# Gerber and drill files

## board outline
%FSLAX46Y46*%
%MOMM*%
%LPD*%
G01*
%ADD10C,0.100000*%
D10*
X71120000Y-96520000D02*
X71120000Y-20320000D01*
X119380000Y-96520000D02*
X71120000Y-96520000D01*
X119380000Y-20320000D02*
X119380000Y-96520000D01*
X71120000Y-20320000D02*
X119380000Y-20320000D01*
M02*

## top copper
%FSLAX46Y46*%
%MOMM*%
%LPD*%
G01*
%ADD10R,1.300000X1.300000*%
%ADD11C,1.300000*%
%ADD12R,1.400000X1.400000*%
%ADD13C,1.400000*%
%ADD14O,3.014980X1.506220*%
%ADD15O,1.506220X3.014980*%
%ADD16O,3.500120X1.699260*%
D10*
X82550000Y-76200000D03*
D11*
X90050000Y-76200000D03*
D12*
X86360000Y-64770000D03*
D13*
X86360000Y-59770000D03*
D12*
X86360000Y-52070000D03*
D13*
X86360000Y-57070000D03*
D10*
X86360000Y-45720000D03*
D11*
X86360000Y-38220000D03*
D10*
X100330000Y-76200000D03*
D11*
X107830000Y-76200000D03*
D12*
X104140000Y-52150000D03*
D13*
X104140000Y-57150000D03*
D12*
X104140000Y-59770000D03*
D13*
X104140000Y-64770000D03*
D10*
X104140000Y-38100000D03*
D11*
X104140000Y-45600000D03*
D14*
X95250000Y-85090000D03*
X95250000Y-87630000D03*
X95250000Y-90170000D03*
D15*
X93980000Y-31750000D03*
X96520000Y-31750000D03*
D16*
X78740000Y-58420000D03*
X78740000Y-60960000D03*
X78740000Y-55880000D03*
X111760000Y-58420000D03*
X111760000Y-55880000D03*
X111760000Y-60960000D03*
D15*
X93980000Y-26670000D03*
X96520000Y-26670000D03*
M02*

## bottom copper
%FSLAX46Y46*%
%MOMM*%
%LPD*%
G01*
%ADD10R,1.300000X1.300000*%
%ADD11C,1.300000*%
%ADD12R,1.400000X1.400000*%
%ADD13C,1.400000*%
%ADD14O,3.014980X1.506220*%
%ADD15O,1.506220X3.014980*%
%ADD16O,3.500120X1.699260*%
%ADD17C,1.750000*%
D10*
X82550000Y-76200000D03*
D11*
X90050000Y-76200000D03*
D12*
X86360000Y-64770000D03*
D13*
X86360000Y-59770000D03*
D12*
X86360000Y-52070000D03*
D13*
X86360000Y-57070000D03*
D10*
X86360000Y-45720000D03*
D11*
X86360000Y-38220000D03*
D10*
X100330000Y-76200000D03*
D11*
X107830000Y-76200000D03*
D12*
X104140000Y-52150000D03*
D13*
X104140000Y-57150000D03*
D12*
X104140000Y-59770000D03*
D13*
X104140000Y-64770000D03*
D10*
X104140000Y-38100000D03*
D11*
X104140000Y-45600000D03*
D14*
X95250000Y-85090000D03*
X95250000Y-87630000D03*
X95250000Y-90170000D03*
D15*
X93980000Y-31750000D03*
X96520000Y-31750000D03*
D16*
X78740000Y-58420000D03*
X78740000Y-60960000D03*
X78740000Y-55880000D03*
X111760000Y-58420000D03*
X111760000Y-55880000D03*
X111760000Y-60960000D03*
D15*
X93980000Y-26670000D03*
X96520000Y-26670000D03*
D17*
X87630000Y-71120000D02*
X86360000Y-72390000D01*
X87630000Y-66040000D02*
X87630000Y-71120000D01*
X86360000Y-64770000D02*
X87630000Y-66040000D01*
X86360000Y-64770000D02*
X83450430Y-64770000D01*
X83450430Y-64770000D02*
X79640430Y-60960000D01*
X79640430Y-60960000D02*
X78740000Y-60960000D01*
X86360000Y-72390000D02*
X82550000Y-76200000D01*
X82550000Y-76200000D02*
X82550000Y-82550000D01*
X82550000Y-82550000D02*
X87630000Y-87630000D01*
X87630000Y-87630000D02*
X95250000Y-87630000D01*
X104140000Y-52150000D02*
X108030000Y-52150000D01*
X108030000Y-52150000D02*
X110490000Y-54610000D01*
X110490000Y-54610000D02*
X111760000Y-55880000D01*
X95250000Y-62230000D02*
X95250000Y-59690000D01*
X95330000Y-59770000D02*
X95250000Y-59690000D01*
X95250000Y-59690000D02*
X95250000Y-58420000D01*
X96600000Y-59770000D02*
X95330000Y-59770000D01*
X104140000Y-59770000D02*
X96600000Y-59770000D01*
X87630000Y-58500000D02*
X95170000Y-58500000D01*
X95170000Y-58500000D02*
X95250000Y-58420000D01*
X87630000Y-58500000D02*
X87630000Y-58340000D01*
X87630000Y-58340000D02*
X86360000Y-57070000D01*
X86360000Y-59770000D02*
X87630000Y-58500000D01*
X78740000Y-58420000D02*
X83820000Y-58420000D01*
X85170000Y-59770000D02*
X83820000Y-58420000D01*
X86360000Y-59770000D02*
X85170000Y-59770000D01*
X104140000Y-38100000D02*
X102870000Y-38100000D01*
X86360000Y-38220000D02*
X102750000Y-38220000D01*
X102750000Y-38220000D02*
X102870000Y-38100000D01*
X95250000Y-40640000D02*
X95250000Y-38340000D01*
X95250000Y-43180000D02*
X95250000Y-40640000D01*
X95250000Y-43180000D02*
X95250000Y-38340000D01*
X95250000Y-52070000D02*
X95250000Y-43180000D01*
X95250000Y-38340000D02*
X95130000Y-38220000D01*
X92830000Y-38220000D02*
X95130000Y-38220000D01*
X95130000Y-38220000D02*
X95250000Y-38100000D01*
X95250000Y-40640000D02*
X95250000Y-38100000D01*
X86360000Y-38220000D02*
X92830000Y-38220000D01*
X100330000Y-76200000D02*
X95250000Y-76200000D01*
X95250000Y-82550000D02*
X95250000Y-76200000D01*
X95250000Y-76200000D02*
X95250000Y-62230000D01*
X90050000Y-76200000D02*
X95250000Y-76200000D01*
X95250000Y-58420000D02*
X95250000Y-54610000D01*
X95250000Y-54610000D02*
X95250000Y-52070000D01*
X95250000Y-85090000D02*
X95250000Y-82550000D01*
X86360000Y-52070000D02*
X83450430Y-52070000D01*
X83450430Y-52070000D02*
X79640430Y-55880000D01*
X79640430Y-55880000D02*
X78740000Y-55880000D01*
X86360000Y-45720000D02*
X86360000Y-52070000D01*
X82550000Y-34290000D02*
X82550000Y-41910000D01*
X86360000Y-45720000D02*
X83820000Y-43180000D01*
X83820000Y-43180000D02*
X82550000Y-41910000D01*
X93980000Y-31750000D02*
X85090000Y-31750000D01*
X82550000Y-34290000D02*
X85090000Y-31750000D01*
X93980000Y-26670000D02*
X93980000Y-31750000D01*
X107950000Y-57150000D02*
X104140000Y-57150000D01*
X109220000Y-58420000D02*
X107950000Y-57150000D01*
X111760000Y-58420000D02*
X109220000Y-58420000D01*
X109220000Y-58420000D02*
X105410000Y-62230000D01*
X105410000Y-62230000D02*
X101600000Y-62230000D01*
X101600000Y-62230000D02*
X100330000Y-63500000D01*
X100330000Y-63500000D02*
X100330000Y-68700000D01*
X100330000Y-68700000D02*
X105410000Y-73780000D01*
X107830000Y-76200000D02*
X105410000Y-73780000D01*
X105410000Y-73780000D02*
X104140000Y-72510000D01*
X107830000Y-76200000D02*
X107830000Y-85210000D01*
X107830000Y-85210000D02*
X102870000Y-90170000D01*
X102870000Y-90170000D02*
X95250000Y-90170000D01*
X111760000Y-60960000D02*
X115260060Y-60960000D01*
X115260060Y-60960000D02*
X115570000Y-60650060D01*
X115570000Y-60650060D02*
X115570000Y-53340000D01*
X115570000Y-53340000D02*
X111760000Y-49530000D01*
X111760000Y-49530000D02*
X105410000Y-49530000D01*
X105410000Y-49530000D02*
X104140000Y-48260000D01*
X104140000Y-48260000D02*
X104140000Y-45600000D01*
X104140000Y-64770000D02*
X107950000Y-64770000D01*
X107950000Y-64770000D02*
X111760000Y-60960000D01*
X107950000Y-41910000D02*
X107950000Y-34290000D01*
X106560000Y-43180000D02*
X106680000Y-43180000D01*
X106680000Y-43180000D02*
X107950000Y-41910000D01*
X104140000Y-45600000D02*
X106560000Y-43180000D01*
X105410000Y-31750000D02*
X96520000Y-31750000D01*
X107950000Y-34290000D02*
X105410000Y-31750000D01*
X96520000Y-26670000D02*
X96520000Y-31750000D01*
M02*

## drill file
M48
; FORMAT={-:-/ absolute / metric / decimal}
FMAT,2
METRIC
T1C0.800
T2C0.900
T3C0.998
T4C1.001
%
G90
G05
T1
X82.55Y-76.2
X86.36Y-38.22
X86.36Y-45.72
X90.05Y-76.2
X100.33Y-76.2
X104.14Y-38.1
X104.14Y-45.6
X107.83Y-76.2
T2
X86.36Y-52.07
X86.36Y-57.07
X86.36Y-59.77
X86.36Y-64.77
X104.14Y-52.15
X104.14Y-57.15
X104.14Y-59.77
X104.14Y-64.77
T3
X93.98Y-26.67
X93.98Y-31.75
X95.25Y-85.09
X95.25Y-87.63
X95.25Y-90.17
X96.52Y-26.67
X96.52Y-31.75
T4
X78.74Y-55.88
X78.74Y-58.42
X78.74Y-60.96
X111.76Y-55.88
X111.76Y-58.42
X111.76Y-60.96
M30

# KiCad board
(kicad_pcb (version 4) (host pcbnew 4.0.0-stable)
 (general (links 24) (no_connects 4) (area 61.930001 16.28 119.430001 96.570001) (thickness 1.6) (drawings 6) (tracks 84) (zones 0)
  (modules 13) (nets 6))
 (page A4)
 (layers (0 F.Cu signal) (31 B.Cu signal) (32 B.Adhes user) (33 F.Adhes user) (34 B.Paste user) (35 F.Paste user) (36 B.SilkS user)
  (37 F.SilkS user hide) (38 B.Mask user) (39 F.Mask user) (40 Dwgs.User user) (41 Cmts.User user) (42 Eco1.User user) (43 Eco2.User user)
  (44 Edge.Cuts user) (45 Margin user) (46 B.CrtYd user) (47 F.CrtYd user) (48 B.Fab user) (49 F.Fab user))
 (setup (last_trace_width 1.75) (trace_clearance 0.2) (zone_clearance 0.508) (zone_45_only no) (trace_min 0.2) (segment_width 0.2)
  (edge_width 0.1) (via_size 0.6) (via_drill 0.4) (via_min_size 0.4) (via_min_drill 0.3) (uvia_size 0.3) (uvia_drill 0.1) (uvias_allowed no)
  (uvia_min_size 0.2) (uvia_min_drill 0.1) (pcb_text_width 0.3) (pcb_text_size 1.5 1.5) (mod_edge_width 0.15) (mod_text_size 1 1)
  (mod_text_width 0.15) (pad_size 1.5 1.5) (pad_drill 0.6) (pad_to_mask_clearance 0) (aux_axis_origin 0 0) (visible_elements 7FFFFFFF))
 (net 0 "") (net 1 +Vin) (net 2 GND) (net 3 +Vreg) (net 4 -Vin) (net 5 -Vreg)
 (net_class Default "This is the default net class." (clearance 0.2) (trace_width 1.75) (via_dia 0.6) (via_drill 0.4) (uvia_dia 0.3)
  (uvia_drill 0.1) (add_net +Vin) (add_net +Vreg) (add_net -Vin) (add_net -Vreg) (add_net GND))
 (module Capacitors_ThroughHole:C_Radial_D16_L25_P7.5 (layer F.Cu) (at 82.55 76.2)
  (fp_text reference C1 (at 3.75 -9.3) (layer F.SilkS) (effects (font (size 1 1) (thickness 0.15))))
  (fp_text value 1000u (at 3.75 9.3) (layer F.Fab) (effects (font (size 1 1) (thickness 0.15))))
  (pad 1 thru_hole rect (at 0 0) (size 1.3 1.3) (drill 0.8) (layers *.Cu *.Mask F.SilkS) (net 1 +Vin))
  (pad 2 thru_hole circle (at 7.5 0) (size 1.3 1.3) (drill 0.8) (layers *.Cu *.Mask F.SilkS) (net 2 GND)))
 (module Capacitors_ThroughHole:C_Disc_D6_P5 (layer F.Cu) (at 86.36 64.77 90)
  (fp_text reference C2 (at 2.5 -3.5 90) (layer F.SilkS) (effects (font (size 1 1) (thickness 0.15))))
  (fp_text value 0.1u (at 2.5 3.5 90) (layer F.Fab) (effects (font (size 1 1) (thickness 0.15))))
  (pad 1 thru_hole rect (at 0 0 90) (size 1.4 1.4) (drill 0.9) (layers *.Cu *.Mask F.SilkS) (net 1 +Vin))
  (pad 2 thru_hole circle (at 5 0 90) (size 1.4 1.4) (drill 0.9) (layers *.Cu *.Mask F.SilkS) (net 2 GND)))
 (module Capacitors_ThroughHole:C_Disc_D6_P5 (layer F.Cu) (at 86.36 52.07 270)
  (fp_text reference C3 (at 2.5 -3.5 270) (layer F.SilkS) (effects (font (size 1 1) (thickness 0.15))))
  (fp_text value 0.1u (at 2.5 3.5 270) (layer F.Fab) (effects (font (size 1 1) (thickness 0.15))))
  (pad 1 thru_hole rect (at 0 0 270) (size 1.4 1.4) (drill 0.9) (layers *.Cu *.Mask F.SilkS) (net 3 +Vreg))
  (pad 2 thru_hole circle (at 5 0 270) (size 1.4 1.4) (drill 0.9) (layers *.Cu *.Mask F.SilkS) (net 2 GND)))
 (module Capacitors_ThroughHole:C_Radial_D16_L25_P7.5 (layer F.Cu) (at 86.36 45.72 90)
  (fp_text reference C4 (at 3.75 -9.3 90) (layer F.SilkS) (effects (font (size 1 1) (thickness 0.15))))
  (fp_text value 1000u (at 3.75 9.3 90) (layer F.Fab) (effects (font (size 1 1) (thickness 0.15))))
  (pad 1 thru_hole rect (at 0 0 90) (size 1.3 1.3) (drill 0.8) (layers *.Cu *.Mask F.SilkS) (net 3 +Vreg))
  (pad 2 thru_hole circle (at 7.5 0 90) (size 1.3 1.3) (drill 0.8) (layers *.Cu *.Mask F.SilkS) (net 2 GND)))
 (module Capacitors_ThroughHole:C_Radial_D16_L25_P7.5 (layer F.Cu) (at 100.33 76.2)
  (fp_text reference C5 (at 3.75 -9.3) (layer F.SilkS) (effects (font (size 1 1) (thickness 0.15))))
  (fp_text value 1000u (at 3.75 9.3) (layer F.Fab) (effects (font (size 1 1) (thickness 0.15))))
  (pad 1 thru_hole rect (at 0 0) (size 1.3 1.3) (drill 0.8) (layers *.Cu *.Mask F.SilkS) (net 2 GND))
  (pad 2 thru_hole circle (at 7.5 0) (size 1.3 1.3) (drill 0.8) (layers *.Cu *.Mask F.SilkS) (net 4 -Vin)))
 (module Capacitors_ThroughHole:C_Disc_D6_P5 (layer F.Cu) (at 104.14 52.15 270)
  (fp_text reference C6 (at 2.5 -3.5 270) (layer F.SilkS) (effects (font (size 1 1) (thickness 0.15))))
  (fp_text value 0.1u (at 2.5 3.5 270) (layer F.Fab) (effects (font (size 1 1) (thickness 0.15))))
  (pad 1 thru_hole rect (at 0 0 270) (size 1.4 1.4) (drill 0.9) (layers *.Cu *.Mask F.SilkS) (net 2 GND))
  (pad 2 thru_hole circle (at 5 0 270) (size 1.4 1.4) (drill 0.9) (layers *.Cu *.Mask F.SilkS) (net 4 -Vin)))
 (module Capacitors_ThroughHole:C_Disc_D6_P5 (layer F.Cu) (at 104.14 59.77 270)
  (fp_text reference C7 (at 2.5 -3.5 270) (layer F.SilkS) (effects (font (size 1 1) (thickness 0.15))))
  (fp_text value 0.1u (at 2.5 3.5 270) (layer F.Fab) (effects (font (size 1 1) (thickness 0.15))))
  (pad 1 thru_hole rect (at 0 0 270) (size 1.4 1.4) (drill 0.9) (layers *.Cu *.Mask F.SilkS) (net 2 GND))
  (pad 2 thru_hole circle (at 5 0 270) (size 1.4 1.4) (drill 0.9) (layers *.Cu *.Mask F.SilkS) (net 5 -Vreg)))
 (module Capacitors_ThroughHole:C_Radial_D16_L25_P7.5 (layer F.Cu) (at 104.14 38.1 270)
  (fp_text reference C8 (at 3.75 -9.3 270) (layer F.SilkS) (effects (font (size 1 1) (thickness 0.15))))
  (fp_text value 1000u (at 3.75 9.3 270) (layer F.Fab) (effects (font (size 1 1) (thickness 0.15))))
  (pad 1 thru_hole rect (at 0 0 270) (size 1.3 1.3) (drill 0.8) (layers *.Cu *.Mask F.SilkS) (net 2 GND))
  (pad 2 thru_hole circle (at 7.5 0 270) (size 1.3 1.3) (drill 0.8) (layers *.Cu *.Mask F.SilkS) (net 5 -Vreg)))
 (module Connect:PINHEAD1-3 (layer F.Cu) (at 95.25 87.63 270)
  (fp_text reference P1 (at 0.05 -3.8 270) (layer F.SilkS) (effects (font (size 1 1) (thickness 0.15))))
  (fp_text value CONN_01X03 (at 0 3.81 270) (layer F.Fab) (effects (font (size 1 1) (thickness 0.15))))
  (pad 1 thru_hole oval (at -2.54 0 270) (size 1.50622 3.01498) (drill 0.99822) (layers *.Cu *.Mask) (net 2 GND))
  (pad 2 thru_hole oval (at 0 0 270) (size 1.50622 3.01498) (drill 0.99822) (layers *.Cu *.Mask) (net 1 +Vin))
  (pad 3 thru_hole oval (at 2.54 0 270) (size 1.50622 3.01498) (drill 0.99822) (layers *.Cu *.Mask) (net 4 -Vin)))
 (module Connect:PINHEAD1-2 (layer F.Cu) (at 95.25 31.75)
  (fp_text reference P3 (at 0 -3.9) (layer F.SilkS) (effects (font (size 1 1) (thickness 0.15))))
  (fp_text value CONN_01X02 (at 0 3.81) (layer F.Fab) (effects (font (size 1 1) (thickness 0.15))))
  (pad 1 thru_hole oval (at -1.27 0) (size 1.50622 3.01498) (drill 0.99822) (layers *.Cu *.Mask) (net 3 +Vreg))
  (pad 2 thru_hole oval (at 1.27 0) (size 1.50622 3.01498) (drill 0.99822) (layers *.Cu *.Mask) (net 5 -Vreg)))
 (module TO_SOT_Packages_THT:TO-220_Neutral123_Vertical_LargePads (layer F.Cu) (at 78.74 58.42 90)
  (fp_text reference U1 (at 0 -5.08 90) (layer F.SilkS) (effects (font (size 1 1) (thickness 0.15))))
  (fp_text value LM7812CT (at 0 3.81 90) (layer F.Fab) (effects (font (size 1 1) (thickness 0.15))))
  (pad 2 thru_hole oval (at 0 0 180) (size 3.50012 1.69926) (drill 1.00076) (layers *.Cu *.Mask F.SilkS) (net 2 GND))
  (pad 1 thru_hole oval (at -2.54 0 180) (size 3.50012 1.69926) (drill 1.00076) (layers *.Cu *.Mask F.SilkS) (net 1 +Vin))
  (pad 3 thru_hole oval (at 2.54 0 180) (size 3.50012 1.69926) (drill 1.00076) (layers *.Cu *.Mask F.SilkS) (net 3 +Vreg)))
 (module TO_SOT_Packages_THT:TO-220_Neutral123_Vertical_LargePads (layer F.Cu) (at 111.76 58.42 270)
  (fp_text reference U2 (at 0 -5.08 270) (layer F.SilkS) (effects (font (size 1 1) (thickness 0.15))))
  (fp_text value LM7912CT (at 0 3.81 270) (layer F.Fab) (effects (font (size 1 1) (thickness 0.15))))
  (pad 2 thru_hole oval (at 0 0) (size 3.50012 1.69926) (drill 1.00076) (layers *.Cu *.Mask F.SilkS) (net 4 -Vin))
  (pad 1 thru_hole oval (at -2.54 0) (size 3.50012 1.69926) (drill 1.00076) (layers *.Cu *.Mask F.SilkS) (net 2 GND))
  (pad 3 thru_hole oval (at 2.54 0) (size 3.50012 1.69926) (drill 1.00076) (layers *.Cu *.Mask F.SilkS) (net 5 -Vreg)))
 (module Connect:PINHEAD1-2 (layer F.Cu) (at 95.25 26.67)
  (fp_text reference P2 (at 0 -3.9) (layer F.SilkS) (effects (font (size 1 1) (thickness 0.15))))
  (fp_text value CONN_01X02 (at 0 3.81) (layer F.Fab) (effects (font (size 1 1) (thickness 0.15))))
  (pad 1 thru_hole oval (at -1.27 0) (size 1.50622 3.01498) (drill 0.99822) (layers *.Cu *.Mask) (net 3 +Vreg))
  (pad 2 thru_hole oval (at 1.27 0) (size 1.50622 3.01498) (drill 0.99822) (layers *.Cu *.Mask) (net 5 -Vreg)))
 (gr_line (start 71.12 96.52) (end 71.12 20.32) (angle 90) (layer Edge.Cuts) (width 0.1))
 (gr_line (start 119.38 96.52) (end 71.12 96.52) (angle 90) (layer Edge.Cuts) (width 0.1))
 (gr_line (start 119.38 20.32) (end 119.38 96.52) (angle 90) (layer Edge.Cuts) (width 0.1))
 (gr_line (start 71.12 20.32) (end 119.38 20.32) (angle 90) (layer Edge.Cuts) (width 0.1))
 (segment (start 87.63 71.12) (end 86.36 72.39) (width 1.75) (layer B.Cu) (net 1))
 (segment (start 87.63 66.04) (end 87.63 71.12) (width 1.75) (layer B.Cu) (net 1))
 (segment (start 86.36 64.77) (end 87.63 66.04) (width 1.75) (layer B.Cu) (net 1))
 (segment (start 86.36 64.77) (end 83.45043 64.77) (width 1.75) (layer B.Cu) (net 1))
 (segment (start 83.45043 64.77) (end 79.64043 60.96) (width 1.75) (layer B.Cu) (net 1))
 (segment (start 79.64043 60.96) (end 78.74 60.96) (width 1.75) (layer B.Cu) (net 1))
 (segment (start 86.36 72.39) (end 82.55 76.2) (width 1.75) (layer B.Cu) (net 1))
 (segment (start 82.55 76.2) (end 82.55 82.55) (width 1.75) (layer B.Cu) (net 1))
 (segment (start 82.55 82.55) (end 87.63 87.63) (width 1.75) (layer B.Cu) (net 1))
 (segment (start 87.63 87.63) (end 95.25 87.63) (width 1.75) (layer B.Cu) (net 1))
 (segment (start 104.14 52.15) (end 108.03 52.15) (width 1.75) (layer B.Cu) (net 2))
 (segment (start 108.03 52.15) (end 110.49 54.61) (width 1.75) (layer B.Cu) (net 2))
 (segment (start 110.49 54.61) (end 111.76 55.88) (width 1.75) (layer B.Cu) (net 2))
 (segment (start 95.25 62.23) (end 95.25 59.69) (width 1.75) (layer B.Cu) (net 2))
 (segment (start 95.33 59.77) (end 95.25 59.69) (width 1.75) (layer B.Cu) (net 2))
 (segment (start 95.25 59.69) (end 95.25 58.42) (width 1.75) (layer B.Cu) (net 2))
 (segment (start 96.6 59.77) (end 95.33 59.77) (width 1.75) (layer B.Cu) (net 2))
 (segment (start 104.14 59.77) (end 96.6 59.77) (width 1.75) (layer B.Cu) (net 2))
 (segment (start 87.63 58.5) (end 95.17 58.5) (width 1.75) (layer B.Cu) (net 2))
 (segment (start 95.17 58.5) (end 95.25 58.42) (width 1.75) (layer B.Cu) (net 2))
 (segment (start 87.63 58.5) (end 87.63 58.34) (width 1.75) (layer B.Cu) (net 2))
 (segment (start 87.63 58.34) (end 86.36 57.07) (width 1.75) (layer B.Cu) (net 2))
 (segment (start 86.36 59.77) (end 87.63 58.5) (width 1.75) (layer B.Cu) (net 2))
 (segment (start 78.74 58.42) (end 83.82 58.42) (width 1.75) (layer B.Cu) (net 2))
 (segment (start 85.17 59.77) (end 83.82 58.42) (width 1.75) (layer B.Cu) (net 2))
 (segment (start 86.36 59.77) (end 85.17 59.77) (width 1.75) (layer B.Cu) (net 2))
 (segment (start 104.14 38.1) (end 102.87 38.1) (width 1.75) (layer B.Cu) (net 2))
 (segment (start 86.36 38.22) (end 102.75 38.22) (width 1.75) (layer B.Cu) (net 2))
 (segment (start 102.75 38.22) (end 102.87 38.1) (width 1.75) (layer B.Cu) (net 2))
 (segment (start 95.25 40.64) (end 95.25 38.34) (width 1.75) (layer B.Cu) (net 2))
 (segment (start 95.25 43.18) (end 95.25 40.64) (width 1.75) (layer B.Cu) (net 2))
 (segment (start 95.25 43.18) (end 95.25 38.34) (width 1.75) (layer B.Cu) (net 2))
 (segment (start 95.25 52.07) (end 95.25 43.18) (width 1.75) (layer B.Cu) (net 2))
 (segment (start 95.25 38.34) (end 95.13 38.22) (width 1.75) (layer B.Cu) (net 2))
 (segment (start 92.83 38.22) (end 95.13 38.22) (width 1.75) (layer B.Cu) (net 2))
 (segment (start 95.13 38.22) (end 95.25 38.1) (width 1.75) (layer B.Cu) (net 2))
 (segment (start 95.25 40.64) (end 95.25 38.1) (width 1.75) (layer B.Cu) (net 2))
 (segment (start 86.36 38.22) (end 92.83 38.22) (width 1.75) (layer B.Cu) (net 2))
 (segment (start 100.33 76.2) (end 95.25 76.2) (width 1.75) (layer B.Cu) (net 2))
 (segment (start 95.25 82.55) (end 95.25 76.2) (width 1.75) (layer B.Cu) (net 2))
 (segment (start 95.25 76.2) (end 95.25 62.23) (width 1.75) (layer B.Cu) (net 2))
 (segment (start 90.05 76.2) (end 95.25 76.2) (width 1.75) (layer B.Cu) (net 2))
 (segment (start 95.25 58.42) (end 95.25 54.61) (width 1.75) (layer B.Cu) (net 2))
 (segment (start 95.25 54.61) (end 95.25 52.07) (width 1.75) (layer B.Cu) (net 2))
 (segment (start 95.25 85.09) (end 95.25 82.55) (width 1.75) (layer B.Cu) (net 2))
 (segment (start 86.36 52.07) (end 83.45043 52.07) (width 1.75) (layer B.Cu) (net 3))
 (segment (start 83.45043 52.07) (end 79.64043 55.88) (width 1.75) (layer B.Cu) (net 3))
 (segment (start 79.64043 55.88) (end 78.74 55.88) (width 1.75) (layer B.Cu) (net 3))
 (segment (start 86.36 45.72) (end 86.36 52.07) (width 1.75) (layer B.Cu) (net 3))
 (segment (start 82.55 34.29) (end 82.55 41.91) (width 1.75) (layer B.Cu) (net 3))
 (segment (start 86.36 45.72) (end 83.82 43.18) (width 1.75) (layer B.Cu) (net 3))
 (segment (start 83.82 43.18) (end 82.55 41.91) (width 1.75) (layer B.Cu) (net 3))
 (segment (start 93.98 31.75) (end 85.09 31.75) (width 1.75) (layer B.Cu) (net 3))
 (segment (start 82.55 34.29) (end 85.09 31.75) (width 1.75) (layer B.Cu) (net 3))
 (segment (start 93.98 26.67) (end 93.98 31.75) (width 1.75) (layer B.Cu) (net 3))
 (segment (start 107.95 57.15) (end 104.14 57.15) (width 1.75) (layer B.Cu) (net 4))
 (segment (start 109.22 58.42) (end 107.95 57.15) (width 1.75) (layer B.Cu) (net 4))
 (segment (start 111.76 58.42) (end 109.22 58.42) (width 1.75) (layer B.Cu) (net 4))
 (segment (start 109.22 58.42) (end 105.41 62.23) (width 1.75) (layer B.Cu) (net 4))
 (segment (start 105.41 62.23) (end 101.6 62.23) (width 1.75) (layer B.Cu) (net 4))
 (segment (start 101.6 62.23) (end 100.33 63.5) (width 1.75) (layer B.Cu) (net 4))
 (segment (start 100.33 63.5) (end 100.33 68.7) (width 1.75) (layer B.Cu) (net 4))
 (segment (start 100.33 68.7) (end 105.41 73.78) (width 1.75) (layer B.Cu) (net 4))
 (segment (start 107.83 76.2) (end 105.41 73.78) (width 1.75) (layer B.Cu) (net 4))
 (segment (start 105.41 73.78) (end 104.14 72.51) (width 1.75) (layer B.Cu) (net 4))
 (segment (start 107.83 76.2) (end 107.83 85.21) (width 1.75) (layer B.Cu) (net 4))
 (segment (start 107.83 85.21) (end 102.87 90.17) (width 1.75) (layer B.Cu) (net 4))
 (segment (start 102.87 90.17) (end 95.25 90.17) (width 1.75) (layer B.Cu) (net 4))
 (segment (start 111.76 60.96) (end 115.26006 60.96) (width 1.75) (layer B.Cu) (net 5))
 (segment (start 115.26006 60.96) (end 115.57 60.65006) (width 1.75) (layer B.Cu) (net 5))
 (segment (start 115.57 60.65006) (end 115.57 53.34) (width 1.75) (layer B.Cu) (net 5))
 (segment (start 115.57 53.34) (end 111.76 49.53) (width 1.75) (layer B.Cu) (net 5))
 (segment (start 111.76 49.53) (end 105.41 49.53) (width 1.75) (layer B.Cu) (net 5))
 (segment (start 105.41 49.53) (end 104.14 48.26) (width 1.75) (layer B.Cu) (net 5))
 (segment (start 104.14 48.26) (end 104.14 45.6) (width 1.75) (layer B.Cu) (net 5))
 (segment (start 104.14 64.77) (end 107.95 64.77) (width 1.75) (layer B.Cu) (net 5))
 (segment (start 107.95 64.77) (end 111.76 60.96) (width 1.75) (layer B.Cu) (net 5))
 (segment (start 107.95 41.91) (end 107.95 34.29) (width 1.75) (layer B.Cu) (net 5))
 (segment (start 106.56 43.18) (end 106.68 43.18) (width 1.75) (layer B.Cu) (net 5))
 (segment (start 106.68 43.18) (end 107.95 41.91) (width 1.75) (layer B.Cu) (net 5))
 (segment (start 104.14 45.6) (end 106.56 43.18) (width 1.75) (layer B.Cu) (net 5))
 (segment (start 105.41 31.75) (end 96.52 31.75) (width 1.75) (layer B.Cu) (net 5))
 (segment (start 107.95 34.29) (end 105.41 31.75) (width 1.75) (layer B.Cu) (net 5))
 (segment (start 96.52 26.67) (end 96.52 31.75) (width 1.75) (layer B.Cu) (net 5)))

